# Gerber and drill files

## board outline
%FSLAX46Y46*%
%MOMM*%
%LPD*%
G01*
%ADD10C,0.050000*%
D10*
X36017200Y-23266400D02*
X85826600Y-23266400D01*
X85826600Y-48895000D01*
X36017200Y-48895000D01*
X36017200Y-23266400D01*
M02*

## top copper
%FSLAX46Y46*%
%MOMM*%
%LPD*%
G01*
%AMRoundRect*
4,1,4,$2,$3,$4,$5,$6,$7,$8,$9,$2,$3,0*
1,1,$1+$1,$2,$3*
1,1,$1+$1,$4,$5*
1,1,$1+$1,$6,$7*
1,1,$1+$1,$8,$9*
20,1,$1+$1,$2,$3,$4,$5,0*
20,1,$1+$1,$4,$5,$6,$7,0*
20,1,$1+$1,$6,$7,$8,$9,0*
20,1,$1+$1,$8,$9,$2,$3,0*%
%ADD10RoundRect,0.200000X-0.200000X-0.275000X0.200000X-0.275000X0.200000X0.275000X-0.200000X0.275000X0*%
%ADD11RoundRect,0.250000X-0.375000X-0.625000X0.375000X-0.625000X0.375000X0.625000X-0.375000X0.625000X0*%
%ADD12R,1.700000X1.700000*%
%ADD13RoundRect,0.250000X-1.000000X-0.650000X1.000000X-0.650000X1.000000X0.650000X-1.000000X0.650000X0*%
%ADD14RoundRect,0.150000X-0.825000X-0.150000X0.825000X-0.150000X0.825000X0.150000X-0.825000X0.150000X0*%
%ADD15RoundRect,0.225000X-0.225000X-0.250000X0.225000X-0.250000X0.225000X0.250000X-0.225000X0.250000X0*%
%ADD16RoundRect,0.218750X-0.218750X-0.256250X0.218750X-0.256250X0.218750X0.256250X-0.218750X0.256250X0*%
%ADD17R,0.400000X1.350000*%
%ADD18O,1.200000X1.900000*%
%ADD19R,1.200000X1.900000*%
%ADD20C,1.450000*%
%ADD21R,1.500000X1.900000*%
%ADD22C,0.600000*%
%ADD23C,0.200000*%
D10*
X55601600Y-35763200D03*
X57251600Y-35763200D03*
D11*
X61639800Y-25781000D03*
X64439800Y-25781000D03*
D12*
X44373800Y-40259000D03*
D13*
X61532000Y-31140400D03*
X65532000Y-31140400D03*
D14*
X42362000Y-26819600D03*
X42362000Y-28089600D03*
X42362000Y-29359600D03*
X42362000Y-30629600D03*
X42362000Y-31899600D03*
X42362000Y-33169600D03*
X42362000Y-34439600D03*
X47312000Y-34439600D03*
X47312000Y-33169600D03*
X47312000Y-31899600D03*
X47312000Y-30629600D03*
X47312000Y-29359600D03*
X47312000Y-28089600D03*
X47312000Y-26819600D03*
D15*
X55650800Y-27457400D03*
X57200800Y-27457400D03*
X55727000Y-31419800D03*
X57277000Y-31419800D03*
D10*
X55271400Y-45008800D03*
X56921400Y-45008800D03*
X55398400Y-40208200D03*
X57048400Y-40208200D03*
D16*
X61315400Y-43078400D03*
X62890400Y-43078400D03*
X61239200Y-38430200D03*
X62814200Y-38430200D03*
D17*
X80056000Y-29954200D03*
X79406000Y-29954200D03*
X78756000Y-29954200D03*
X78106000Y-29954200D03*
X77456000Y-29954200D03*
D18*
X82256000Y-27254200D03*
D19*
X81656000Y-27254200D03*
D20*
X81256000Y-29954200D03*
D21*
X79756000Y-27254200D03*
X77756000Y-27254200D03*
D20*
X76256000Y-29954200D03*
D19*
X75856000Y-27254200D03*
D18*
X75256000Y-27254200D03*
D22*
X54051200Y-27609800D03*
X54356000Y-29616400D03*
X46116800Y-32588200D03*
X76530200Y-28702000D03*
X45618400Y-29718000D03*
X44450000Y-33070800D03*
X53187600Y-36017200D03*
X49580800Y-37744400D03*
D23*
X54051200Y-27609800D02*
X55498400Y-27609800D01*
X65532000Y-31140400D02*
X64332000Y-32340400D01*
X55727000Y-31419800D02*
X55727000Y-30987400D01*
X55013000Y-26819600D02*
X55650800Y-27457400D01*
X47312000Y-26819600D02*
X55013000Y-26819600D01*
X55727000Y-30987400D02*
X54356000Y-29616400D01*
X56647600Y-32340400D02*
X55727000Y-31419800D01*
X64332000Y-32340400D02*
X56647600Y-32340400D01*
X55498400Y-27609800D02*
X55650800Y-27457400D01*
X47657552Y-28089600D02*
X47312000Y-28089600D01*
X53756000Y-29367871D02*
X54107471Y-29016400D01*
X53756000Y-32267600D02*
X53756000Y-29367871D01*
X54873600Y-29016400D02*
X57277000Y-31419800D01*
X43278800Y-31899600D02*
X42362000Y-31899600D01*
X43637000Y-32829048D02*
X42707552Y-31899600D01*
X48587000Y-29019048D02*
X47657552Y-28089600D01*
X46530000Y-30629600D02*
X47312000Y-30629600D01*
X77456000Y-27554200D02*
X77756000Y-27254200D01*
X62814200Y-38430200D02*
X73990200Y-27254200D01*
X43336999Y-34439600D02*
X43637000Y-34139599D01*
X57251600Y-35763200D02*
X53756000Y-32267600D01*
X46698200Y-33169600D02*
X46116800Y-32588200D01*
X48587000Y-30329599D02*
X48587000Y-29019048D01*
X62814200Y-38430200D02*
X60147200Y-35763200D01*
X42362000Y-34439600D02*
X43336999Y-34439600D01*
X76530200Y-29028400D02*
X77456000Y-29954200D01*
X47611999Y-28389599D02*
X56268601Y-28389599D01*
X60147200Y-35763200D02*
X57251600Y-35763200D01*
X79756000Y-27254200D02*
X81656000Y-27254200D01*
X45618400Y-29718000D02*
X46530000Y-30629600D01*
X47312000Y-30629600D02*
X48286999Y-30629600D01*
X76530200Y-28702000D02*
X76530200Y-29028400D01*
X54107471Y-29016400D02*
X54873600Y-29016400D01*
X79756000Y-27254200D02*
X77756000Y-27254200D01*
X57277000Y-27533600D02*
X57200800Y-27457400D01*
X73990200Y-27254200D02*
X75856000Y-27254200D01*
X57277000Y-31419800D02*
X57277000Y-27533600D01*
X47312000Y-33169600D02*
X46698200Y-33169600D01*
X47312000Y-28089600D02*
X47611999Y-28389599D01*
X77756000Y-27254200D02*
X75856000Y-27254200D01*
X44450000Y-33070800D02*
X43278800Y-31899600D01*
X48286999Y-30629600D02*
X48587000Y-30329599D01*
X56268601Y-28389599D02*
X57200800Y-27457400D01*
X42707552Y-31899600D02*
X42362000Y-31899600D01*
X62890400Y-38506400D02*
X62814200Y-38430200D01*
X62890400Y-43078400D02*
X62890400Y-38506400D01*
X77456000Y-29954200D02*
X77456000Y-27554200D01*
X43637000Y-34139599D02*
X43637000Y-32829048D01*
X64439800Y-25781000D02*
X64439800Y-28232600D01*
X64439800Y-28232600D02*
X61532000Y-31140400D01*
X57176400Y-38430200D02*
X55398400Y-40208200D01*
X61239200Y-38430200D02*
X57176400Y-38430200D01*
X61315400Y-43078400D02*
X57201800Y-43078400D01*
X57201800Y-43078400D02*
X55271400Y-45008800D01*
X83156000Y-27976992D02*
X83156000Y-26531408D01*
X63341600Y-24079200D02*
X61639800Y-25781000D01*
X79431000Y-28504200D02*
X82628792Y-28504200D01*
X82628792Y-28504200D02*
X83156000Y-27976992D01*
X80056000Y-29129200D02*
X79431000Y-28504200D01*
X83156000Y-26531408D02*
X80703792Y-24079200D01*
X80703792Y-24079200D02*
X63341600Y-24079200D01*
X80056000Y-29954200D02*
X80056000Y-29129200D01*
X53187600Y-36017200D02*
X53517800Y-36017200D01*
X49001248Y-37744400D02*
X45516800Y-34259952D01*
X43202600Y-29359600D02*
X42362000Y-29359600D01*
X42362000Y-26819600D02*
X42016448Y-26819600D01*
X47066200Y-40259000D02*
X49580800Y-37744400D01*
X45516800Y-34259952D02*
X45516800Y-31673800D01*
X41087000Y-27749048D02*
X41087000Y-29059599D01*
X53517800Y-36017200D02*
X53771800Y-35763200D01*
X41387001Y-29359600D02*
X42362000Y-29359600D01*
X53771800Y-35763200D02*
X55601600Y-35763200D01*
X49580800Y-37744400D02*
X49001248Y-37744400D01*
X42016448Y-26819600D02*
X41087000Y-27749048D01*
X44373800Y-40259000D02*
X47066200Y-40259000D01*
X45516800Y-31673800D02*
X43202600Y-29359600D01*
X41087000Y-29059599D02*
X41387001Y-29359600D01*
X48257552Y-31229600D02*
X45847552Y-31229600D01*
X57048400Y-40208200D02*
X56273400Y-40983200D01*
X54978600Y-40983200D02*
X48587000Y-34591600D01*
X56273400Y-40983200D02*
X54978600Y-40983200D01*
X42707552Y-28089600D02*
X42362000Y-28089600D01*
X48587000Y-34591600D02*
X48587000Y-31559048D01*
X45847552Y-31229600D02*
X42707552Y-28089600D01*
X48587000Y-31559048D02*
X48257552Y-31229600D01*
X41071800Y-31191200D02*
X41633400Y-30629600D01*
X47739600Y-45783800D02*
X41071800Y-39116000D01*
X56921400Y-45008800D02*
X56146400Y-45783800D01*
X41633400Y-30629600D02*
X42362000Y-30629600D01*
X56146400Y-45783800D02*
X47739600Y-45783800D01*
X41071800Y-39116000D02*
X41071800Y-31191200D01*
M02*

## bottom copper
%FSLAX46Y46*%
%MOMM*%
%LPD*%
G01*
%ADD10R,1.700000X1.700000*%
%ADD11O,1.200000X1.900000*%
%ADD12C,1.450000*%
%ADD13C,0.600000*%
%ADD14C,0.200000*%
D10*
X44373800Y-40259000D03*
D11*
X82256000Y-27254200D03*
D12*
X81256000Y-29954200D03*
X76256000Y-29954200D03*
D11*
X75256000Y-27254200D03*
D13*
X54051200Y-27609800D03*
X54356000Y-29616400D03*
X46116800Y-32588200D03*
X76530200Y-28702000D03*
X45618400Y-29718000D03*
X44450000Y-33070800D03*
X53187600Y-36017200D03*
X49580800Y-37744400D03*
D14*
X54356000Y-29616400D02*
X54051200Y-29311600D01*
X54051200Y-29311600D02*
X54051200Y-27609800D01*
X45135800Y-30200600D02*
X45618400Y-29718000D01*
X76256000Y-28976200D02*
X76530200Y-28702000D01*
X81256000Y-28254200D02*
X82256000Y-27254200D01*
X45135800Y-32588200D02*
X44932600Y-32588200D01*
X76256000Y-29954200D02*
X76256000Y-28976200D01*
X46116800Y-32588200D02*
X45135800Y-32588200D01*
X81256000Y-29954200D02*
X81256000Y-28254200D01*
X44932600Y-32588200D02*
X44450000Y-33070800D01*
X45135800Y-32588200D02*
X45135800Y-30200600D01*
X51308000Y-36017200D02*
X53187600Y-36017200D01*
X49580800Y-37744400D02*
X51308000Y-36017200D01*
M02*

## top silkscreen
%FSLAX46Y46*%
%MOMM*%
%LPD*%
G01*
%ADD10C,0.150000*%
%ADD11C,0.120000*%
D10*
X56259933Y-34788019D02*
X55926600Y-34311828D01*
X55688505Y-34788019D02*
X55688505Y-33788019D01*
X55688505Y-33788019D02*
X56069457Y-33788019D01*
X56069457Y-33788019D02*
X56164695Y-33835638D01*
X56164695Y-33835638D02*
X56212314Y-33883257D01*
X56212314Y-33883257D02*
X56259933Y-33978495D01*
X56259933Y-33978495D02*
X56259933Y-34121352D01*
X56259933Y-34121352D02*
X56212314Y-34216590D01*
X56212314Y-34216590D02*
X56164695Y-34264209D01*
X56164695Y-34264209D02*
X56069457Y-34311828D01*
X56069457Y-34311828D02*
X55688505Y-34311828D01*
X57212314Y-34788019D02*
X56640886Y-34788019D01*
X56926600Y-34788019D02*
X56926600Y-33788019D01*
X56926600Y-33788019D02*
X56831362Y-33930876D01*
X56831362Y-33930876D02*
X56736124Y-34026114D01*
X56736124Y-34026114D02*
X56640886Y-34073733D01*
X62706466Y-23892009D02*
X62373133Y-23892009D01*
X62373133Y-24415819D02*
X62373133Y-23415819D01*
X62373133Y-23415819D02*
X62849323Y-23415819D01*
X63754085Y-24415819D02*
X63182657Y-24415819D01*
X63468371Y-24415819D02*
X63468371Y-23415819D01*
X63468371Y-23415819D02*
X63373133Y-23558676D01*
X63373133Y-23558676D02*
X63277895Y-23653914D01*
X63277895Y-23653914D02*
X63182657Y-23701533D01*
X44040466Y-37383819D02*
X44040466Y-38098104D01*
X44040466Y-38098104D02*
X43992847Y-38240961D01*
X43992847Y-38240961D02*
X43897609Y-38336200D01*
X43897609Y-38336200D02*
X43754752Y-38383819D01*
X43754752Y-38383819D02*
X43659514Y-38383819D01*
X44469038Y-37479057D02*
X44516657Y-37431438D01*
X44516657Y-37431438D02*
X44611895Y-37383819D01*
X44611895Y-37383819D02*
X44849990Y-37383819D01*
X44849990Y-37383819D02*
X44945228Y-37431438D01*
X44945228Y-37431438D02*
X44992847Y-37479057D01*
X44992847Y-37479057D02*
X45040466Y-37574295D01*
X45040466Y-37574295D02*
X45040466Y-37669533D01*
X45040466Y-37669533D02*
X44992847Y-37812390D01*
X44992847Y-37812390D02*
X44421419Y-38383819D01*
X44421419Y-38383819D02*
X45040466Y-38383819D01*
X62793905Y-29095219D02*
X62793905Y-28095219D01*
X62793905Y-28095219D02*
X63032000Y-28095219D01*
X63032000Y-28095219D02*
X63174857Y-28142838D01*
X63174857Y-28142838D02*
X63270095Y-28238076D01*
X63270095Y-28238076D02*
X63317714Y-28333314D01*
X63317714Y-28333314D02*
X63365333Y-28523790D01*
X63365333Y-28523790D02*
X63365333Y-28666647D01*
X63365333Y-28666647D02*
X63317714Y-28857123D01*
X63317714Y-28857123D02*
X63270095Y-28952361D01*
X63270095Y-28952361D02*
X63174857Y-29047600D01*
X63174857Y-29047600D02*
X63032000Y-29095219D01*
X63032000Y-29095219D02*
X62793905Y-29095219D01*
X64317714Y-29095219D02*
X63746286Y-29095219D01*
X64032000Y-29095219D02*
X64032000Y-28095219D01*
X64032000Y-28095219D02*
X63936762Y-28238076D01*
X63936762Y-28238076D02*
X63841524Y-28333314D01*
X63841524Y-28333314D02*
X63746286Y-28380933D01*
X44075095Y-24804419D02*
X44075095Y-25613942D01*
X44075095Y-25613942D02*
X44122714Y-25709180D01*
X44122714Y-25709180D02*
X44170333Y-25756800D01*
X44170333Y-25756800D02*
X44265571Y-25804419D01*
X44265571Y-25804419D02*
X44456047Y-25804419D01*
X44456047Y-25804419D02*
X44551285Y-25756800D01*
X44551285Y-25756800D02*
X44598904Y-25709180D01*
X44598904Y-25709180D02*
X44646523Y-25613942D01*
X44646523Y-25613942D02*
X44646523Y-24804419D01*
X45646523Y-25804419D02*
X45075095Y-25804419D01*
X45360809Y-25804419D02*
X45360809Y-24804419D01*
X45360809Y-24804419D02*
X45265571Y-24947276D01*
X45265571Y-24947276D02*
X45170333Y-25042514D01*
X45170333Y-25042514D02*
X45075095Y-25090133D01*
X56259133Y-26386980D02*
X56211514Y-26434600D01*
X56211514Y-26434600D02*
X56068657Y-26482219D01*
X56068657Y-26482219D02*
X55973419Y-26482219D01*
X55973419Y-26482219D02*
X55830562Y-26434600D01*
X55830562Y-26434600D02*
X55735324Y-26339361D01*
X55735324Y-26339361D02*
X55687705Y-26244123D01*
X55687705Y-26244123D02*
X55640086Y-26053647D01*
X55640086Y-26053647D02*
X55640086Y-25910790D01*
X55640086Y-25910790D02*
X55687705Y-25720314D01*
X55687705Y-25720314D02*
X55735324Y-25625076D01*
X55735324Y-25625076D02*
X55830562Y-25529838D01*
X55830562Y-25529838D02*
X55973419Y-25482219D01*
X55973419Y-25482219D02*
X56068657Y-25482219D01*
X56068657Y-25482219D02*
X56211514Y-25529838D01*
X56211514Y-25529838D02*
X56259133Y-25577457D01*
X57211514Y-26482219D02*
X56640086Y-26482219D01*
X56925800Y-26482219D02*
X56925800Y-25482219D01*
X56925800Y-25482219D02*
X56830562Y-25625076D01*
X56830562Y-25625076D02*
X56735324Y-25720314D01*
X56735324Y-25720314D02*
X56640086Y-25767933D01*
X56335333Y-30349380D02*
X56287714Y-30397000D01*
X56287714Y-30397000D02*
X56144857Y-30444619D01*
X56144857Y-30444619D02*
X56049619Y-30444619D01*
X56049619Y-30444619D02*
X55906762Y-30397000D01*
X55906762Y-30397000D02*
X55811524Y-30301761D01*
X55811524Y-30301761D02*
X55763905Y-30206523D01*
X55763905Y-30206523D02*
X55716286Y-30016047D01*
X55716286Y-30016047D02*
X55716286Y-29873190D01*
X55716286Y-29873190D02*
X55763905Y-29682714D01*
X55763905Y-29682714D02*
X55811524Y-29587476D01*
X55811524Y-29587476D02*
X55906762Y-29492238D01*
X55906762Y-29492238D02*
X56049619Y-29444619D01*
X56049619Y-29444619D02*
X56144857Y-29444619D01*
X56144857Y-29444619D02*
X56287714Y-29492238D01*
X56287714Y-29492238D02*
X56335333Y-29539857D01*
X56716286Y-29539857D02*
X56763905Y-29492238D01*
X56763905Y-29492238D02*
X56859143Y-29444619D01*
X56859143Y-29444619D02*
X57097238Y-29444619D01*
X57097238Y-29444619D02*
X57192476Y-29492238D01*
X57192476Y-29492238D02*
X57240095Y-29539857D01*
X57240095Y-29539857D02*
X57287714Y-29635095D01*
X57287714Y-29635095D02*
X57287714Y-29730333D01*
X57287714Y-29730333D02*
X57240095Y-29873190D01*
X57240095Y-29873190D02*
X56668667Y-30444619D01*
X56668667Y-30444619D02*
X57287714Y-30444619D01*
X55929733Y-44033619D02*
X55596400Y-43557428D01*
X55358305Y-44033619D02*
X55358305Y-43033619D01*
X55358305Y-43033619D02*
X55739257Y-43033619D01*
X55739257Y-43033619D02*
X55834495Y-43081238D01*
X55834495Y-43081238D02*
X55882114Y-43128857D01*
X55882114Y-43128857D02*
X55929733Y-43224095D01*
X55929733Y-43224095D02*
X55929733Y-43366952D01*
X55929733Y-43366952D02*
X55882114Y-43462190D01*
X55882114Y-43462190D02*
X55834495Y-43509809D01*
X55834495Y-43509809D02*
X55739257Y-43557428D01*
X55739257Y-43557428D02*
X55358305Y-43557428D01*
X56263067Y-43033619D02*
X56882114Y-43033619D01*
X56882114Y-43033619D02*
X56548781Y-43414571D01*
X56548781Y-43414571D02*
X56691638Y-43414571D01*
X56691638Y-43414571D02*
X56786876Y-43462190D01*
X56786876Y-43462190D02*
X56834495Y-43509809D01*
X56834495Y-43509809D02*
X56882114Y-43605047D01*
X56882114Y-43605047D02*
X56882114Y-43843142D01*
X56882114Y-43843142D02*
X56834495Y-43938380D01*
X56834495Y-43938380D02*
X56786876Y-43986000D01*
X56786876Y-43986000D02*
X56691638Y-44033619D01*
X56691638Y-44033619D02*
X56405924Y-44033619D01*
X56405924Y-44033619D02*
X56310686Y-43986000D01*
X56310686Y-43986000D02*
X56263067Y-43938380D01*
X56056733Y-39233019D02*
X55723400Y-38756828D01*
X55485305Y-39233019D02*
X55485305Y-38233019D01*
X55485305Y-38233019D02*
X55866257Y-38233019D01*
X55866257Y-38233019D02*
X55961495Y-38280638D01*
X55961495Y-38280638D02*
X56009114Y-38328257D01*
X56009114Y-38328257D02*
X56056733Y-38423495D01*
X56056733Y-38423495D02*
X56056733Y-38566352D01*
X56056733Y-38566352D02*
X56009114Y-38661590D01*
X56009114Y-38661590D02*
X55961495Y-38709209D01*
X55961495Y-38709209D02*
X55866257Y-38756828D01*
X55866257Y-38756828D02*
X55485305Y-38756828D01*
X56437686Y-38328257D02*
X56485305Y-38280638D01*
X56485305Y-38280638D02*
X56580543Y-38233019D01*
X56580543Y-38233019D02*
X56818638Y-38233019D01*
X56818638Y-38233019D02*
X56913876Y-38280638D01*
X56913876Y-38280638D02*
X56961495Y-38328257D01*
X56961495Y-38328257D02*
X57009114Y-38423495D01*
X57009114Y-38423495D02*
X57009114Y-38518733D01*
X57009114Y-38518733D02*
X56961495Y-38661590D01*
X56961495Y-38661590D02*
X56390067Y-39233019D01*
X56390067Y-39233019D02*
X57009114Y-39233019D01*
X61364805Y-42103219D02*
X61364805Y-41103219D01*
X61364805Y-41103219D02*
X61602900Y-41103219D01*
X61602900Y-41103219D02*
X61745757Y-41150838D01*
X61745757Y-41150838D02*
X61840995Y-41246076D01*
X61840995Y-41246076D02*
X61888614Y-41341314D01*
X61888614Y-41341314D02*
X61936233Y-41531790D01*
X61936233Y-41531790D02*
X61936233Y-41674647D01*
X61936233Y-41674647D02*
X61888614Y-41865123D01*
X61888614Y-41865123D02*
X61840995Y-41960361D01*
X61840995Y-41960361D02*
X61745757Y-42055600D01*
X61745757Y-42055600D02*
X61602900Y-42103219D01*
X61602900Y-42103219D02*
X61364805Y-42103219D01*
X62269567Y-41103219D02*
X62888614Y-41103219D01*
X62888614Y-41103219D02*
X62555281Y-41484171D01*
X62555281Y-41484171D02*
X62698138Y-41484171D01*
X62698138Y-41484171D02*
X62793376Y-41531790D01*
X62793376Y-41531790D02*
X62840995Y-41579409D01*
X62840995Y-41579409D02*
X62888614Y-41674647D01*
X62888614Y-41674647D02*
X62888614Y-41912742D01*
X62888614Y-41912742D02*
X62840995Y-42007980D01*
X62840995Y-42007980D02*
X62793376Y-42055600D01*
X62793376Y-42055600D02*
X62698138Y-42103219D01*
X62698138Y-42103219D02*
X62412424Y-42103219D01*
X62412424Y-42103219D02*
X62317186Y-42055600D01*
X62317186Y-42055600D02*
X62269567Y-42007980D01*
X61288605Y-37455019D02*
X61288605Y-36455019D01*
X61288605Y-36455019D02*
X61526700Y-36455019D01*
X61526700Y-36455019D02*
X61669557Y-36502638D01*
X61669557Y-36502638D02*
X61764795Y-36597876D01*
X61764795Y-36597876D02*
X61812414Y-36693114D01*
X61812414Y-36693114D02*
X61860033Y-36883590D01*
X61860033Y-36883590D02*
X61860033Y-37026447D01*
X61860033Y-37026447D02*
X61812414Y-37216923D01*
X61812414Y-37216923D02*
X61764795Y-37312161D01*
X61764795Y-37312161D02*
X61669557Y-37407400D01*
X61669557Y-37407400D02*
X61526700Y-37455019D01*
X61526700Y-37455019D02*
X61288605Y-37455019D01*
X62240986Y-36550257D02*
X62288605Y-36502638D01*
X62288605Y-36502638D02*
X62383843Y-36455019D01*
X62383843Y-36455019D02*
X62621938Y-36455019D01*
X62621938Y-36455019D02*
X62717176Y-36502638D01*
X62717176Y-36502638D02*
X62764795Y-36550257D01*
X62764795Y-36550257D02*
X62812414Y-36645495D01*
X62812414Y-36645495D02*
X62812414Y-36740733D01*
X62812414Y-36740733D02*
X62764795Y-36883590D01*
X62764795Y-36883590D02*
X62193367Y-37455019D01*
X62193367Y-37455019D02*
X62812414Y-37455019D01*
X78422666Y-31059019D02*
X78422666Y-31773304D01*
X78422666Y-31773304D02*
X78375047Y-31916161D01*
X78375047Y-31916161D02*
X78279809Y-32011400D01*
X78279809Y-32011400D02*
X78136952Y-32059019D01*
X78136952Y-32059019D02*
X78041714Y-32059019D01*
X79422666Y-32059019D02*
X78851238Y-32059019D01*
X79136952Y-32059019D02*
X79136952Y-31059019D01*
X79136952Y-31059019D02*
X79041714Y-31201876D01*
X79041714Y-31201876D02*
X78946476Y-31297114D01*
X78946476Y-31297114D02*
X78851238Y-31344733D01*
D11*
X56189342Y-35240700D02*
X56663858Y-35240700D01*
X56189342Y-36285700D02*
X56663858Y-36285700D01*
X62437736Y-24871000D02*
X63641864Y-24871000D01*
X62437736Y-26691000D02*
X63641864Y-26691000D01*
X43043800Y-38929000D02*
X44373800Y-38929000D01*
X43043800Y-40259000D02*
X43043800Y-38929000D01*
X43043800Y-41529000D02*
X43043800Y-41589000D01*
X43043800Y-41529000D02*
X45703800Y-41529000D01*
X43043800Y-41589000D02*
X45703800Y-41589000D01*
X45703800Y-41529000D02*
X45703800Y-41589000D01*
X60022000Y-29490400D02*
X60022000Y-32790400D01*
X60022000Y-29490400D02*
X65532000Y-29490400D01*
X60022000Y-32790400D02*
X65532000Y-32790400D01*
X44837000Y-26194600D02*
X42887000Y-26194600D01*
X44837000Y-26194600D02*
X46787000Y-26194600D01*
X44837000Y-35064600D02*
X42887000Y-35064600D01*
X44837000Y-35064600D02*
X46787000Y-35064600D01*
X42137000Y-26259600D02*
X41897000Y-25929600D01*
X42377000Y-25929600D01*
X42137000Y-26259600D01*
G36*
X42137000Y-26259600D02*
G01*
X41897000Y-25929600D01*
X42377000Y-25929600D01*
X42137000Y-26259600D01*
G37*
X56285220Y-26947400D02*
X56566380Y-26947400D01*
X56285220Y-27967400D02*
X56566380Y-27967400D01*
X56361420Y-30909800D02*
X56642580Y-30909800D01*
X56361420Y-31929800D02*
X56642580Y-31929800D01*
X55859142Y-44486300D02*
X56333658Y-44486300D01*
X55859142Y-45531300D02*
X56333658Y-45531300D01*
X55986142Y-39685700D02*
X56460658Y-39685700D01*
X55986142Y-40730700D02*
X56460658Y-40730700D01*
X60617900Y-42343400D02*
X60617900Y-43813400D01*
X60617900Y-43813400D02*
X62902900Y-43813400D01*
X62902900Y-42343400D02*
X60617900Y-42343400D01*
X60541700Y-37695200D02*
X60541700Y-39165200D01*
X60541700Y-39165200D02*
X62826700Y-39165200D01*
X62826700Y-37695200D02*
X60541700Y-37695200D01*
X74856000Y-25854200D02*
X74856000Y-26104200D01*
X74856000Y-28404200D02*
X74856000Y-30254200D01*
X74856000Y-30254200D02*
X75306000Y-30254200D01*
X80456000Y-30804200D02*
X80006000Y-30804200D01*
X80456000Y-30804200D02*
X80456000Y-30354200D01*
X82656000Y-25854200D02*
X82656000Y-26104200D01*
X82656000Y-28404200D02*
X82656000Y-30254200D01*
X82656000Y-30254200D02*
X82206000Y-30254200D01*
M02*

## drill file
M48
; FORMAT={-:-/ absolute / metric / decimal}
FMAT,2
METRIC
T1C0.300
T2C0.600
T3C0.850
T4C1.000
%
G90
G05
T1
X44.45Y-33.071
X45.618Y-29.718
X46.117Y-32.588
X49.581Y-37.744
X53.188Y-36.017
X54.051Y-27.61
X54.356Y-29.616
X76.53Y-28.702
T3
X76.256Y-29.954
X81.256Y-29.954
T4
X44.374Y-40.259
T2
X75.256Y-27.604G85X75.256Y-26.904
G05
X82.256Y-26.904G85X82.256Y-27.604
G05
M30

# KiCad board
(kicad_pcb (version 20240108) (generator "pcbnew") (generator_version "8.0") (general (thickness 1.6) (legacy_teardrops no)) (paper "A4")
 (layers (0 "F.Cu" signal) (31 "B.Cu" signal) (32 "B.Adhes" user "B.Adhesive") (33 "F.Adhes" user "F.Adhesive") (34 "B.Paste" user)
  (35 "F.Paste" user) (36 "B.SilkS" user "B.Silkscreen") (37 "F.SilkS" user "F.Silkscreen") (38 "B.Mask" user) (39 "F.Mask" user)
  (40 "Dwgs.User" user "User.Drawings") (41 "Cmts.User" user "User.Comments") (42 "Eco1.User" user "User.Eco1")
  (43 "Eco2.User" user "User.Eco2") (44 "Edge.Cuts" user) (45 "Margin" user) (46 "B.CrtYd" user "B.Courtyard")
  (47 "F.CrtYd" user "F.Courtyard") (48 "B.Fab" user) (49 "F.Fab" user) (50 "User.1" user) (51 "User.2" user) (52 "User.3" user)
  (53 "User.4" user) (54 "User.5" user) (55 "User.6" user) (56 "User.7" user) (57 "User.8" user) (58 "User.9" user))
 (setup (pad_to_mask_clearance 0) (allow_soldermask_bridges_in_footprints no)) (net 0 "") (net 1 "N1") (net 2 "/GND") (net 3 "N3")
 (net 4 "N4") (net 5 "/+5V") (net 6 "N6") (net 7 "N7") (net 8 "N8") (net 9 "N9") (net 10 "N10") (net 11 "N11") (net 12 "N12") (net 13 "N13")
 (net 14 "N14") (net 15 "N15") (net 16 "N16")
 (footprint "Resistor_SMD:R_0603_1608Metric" (layer "F.Cu") (at 56.4266 35.7632)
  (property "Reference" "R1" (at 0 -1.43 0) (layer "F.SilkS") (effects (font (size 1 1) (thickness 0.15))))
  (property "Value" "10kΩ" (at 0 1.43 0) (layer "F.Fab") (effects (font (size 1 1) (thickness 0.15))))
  (fp_line (start -0.237258 -0.5225) (end 0.237258 -0.5225) (stroke (width 0.12) (type solid)) (layer "F.SilkS"))
  (fp_line (start -0.237258 0.5225) (end 0.237258 0.5225) (stroke (width 0.12) (type solid)) (layer "F.SilkS"))
  (pad "1" smd roundrect (at -0.825 0) (size 0.8 0.95) (layers "F.Cu" "F.Paste" "F.Mask") (roundrect_rratio 0.25) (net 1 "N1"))
  (pad "2" smd roundrect (at 0.825 0) (size 0.8 0.95) (layers "F.Cu" "F.Paste" "F.Mask") (roundrect_rratio 0.25) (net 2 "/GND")))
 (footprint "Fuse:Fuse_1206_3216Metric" (layer "F.Cu") (at 63.0398 25.781)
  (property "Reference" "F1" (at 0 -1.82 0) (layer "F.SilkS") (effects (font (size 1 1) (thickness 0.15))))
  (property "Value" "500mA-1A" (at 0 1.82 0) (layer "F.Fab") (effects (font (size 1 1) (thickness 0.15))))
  (fp_line (start -0.602064 -0.91) (end 0.602064 -0.91) (stroke (width 0.12) (type solid)) (layer "F.SilkS"))
  (fp_line (start -0.602064 0.91) (end 0.602064 0.91) (stroke (width 0.12) (type solid)) (layer "F.SilkS"))
  (pad "1" smd roundrect (at -1.4 0) (size 1.25 1.75) (layers "F.Cu" "F.Paste" "F.Mask") (roundrect_rratio 0.2) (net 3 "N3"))
  (pad "2" smd roundrect (at 1.4 0) (size 1.25 1.75) (layers "F.Cu" "F.Paste" "F.Mask") (roundrect_rratio 0.2) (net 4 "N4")))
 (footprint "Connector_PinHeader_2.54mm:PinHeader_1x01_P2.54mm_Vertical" (layer "F.Cu") (at 44.3738 40.259)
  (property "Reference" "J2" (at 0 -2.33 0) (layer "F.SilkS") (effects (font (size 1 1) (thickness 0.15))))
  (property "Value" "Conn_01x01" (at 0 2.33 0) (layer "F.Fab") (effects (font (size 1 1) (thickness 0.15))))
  (fp_line (start -1.33 -1.33) (end 0 -1.33) (stroke (width 0.12) (type solid)) (layer "F.SilkS"))
  (fp_line (start -1.33 0) (end -1.33 -1.33) (stroke (width 0.12) (type solid)) (layer "F.SilkS"))
  (fp_line (start -1.33 1.27) (end -1.33 1.33) (stroke (width 0.12) (type solid)) (layer "F.SilkS"))
  (fp_line (start -1.33 1.27) (end 1.33 1.27) (stroke (width 0.12) (type solid)) (layer "F.SilkS"))
  (fp_line (start -1.33 1.33) (end 1.33 1.33) (stroke (width 0.12) (type solid)) (layer "F.SilkS"))
  (fp_line (start 1.33 1.27) (end 1.33 1.33) (stroke (width 0.12) (type solid)) (layer "F.SilkS"))
  (pad "1" thru_hole rect (at 0 0) (size 1.7 1.7) (drill 1) (layers "*.Cu" "*.Mask") (remove_unused_layers no) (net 1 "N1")))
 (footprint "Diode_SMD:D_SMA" (layer "F.Cu") (at 63.532 31.1404)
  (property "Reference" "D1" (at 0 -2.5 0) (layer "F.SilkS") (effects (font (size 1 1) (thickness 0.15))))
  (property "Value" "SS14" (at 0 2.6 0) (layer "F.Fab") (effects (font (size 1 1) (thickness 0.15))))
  (fp_line (start -3.51 -1.65) (end -3.51 1.65) (stroke (width 0.12) (type solid)) (layer "F.SilkS"))
  (fp_line (start -3.51 -1.65) (end 2 -1.65) (stroke (width 0.12) (type solid)) (layer "F.SilkS"))
  (fp_line (start -3.51 1.65) (end 2 1.65) (stroke (width 0.12) (type solid)) (layer "F.SilkS"))
  (pad "1" smd roundrect (at -2 0) (size 2.5 1.8) (layers "F.Cu" "F.Paste" "F.Mask") (roundrect_rratio 0.1388888889) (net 4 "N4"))
  (pad "2" smd roundrect (at 2 0) (size 2.5 1.8) (layers "F.Cu" "F.Paste" "F.Mask") (roundrect_rratio 0.1388888889) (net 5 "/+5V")))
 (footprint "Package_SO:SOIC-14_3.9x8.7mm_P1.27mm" (layer "F.Cu") (at 44.837 30.6296)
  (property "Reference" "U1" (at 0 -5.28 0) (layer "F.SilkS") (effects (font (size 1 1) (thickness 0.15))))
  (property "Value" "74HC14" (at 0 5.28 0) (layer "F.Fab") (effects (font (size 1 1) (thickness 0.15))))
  (fp_line (start 0 -4.435) (end -1.95 -4.435) (stroke (width 0.12) (type solid)) (layer "F.SilkS"))
  (fp_line (start 0 -4.435) (end 1.95 -4.435) (stroke (width 0.12) (type solid)) (layer "F.SilkS"))
  (fp_line (start 0 4.435) (end -1.95 4.435) (stroke (width 0.12) (type solid)) (layer "F.SilkS"))
  (fp_line (start 0 4.435) (end 1.95 4.435) (stroke (width 0.12) (type solid)) (layer "F.SilkS"))
  (fp_poly
   (pts (xy -2.7 -4.37) (xy -2.94 -4.7) (xy -2.46 -4.7) (xy -2.7 -4.37)) (stroke (width 0.12) (type solid)) (fill solid) (layer "F.SilkS"))
  (pad "1" smd roundrect (at -2.475 -3.81) (size 1.95 0.6) (layers "F.Cu" "F.Paste" "F.Mask") (roundrect_rratio 0.25) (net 1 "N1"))
  (pad "2" smd roundrect (at -2.475 -2.54) (size 1.95 0.6) (layers "F.Cu" "F.Paste" "F.Mask") (roundrect_rratio 0.25) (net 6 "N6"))
  (pad "3" smd roundrect (at -2.475 -1.27) (size 1.95 0.6) (layers "F.Cu" "F.Paste" "F.Mask") (roundrect_rratio 0.25) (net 1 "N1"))
  (pad "4" smd roundrect (at -2.475 0) (size 1.95 0.6) (layers "F.Cu" "F.Paste" "F.Mask") (roundrect_rratio 0.25) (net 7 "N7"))
  (pad "5" smd roundrect (at -2.475 1.27) (size 1.95 0.6) (layers "F.Cu" "F.Paste" "F.Mask") (roundrect_rratio 0.25) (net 2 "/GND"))
  (pad "6" smd roundrect (at -2.475 2.54) (size 1.95 0.6) (layers "F.Cu" "F.Paste" "F.Mask") (roundrect_rratio 0.25) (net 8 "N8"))
  (pad "7" smd roundrect (at -2.475 3.81) (size 1.95 0.6) (layers "F.Cu" "F.Paste" "F.Mask") (roundrect_rratio 0.25) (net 2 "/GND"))
  (pad "8" smd roundrect (at 2.475 3.81) (size 1.95 0.6) (layers "F.Cu" "F.Paste" "F.Mask") (roundrect_rratio 0.25) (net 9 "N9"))
  (pad "9" smd roundrect (at 2.475 2.54) (size 1.95 0.6) (layers "F.Cu" "F.Paste" "F.Mask") (roundrect_rratio 0.25) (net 2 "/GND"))
  (pad "10" smd roundrect (at 2.475 1.27) (size 1.95 0.6) (layers "F.Cu" "F.Paste" "F.Mask") (roundrect_rratio 0.25) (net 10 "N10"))
  (pad "11" smd roundrect (at 2.475 0) (size 1.95 0.6) (layers "F.Cu" "F.Paste" "F.Mask") (roundrect_rratio 0.25) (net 2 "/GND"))
  (pad "12" smd roundrect (at 2.475 -1.27) (size 1.95 0.6) (layers "F.Cu" "F.Paste" "F.Mask") (roundrect_rratio 0.25) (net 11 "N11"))
  (pad "13" smd roundrect (at 2.475 -2.54) (size 1.95 0.6) (layers "F.Cu" "F.Paste" "F.Mask") (roundrect_rratio 0.25) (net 2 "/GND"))
  (pad "14" smd roundrect (at 2.475 -3.81) (size 1.95 0.6) (layers "F.Cu" "F.Paste" "F.Mask") (roundrect_rratio 0.25) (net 5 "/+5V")))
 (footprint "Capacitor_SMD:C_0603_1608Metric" (layer "F.Cu") (at 56.4258 27.4574)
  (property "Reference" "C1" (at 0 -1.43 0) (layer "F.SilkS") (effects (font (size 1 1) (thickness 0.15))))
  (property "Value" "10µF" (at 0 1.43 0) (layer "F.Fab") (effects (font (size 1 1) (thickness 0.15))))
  (fp_line (start -0.14058 -0.51) (end 0.14058 -0.51) (stroke (width 0.12) (type solid)) (layer "F.SilkS"))
  (fp_line (start -0.14058 0.51) (end 0.14058 0.51) (stroke (width 0.12) (type solid)) (layer "F.SilkS"))
  (pad "1" smd roundrect (at -0.775 0) (size 0.9 0.95) (layers "F.Cu" "F.Paste" "F.Mask") (roundrect_rratio 0.25) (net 5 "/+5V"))
  (pad "2" smd roundrect (at 0.775 0) (size 0.9 0.95) (layers "F.Cu" "F.Paste" "F.Mask") (roundrect_rratio 0.25) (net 2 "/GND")))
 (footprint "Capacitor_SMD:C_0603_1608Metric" (layer "F.Cu") (at 56.502 31.4198)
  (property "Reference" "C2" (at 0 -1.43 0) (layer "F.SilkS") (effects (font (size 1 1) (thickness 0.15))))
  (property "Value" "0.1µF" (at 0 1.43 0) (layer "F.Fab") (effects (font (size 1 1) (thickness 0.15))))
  (fp_line (start -0.14058 -0.51) (end 0.14058 -0.51) (stroke (width 0.12) (type solid)) (layer "F.SilkS"))
  (fp_line (start -0.14058 0.51) (end 0.14058 0.51) (stroke (width 0.12) (type solid)) (layer "F.SilkS"))
  (pad "1" smd roundrect (at -0.775 0) (size 0.9 0.95) (layers "F.Cu" "F.Paste" "F.Mask") (roundrect_rratio 0.25) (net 5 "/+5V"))
  (pad "2" smd roundrect (at 0.775 0) (size 0.9 0.95) (layers "F.Cu" "F.Paste" "F.Mask") (roundrect_rratio 0.25) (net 2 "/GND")))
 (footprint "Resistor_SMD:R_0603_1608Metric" (layer "F.Cu") (at 56.0964 45.0088)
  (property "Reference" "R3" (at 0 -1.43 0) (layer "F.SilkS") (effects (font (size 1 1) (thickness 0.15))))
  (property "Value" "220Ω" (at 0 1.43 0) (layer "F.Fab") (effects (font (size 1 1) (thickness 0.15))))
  (fp_line (start -0.237258 -0.5225) (end 0.237258 -0.5225) (stroke (width 0.12) (type solid)) (layer "F.SilkS"))
  (fp_line (start -0.237258 0.5225) (end 0.237258 0.5225) (stroke (width 0.12) (type solid)) (layer "F.SilkS"))
  (pad "1" smd roundrect (at -0.825 0) (size 0.8 0.95) (layers "F.Cu" "F.Paste" "F.Mask") (roundrect_rratio 0.25) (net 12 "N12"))
  (pad "2" smd roundrect (at 0.825 0) (size 0.8 0.95) (layers "F.Cu" "F.Paste" "F.Mask") (roundrect_rratio 0.25) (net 7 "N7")))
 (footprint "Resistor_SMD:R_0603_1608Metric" (layer "F.Cu") (at 56.2234 40.2082)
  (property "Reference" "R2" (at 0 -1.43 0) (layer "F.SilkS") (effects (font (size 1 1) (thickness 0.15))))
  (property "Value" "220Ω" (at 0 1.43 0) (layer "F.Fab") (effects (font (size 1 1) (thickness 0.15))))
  (fp_line (start -0.237258 -0.5225) (end 0.237258 -0.5225) (stroke (width 0.12) (type solid)) (layer "F.SilkS"))
  (fp_line (start -0.237258 0.5225) (end 0.237258 0.5225) (stroke (width 0.12) (type solid)) (layer "F.SilkS"))
  (pad "1" smd roundrect (at -0.825 0) (size 0.8 0.95) (layers "F.Cu" "F.Paste" "F.Mask") (roundrect_rratio 0.25) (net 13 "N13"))
  (pad "2" smd roundrect (at 0.825 0) (size 0.8 0.95) (layers "F.Cu" "F.Paste" "F.Mask") (roundrect_rratio 0.25) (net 6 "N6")))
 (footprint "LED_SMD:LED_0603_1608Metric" (layer "F.Cu") (at 62.1029 43.0784)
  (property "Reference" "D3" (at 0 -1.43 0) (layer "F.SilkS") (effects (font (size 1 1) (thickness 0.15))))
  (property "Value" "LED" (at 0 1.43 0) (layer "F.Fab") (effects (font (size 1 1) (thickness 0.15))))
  (fp_line (start -1.485 -0.735) (end -1.485 0.735) (stroke (width 0.12) (type solid)) (layer "F.SilkS"))
  (fp_line (start -1.485 0.735) (end 0.8 0.735) (stroke (width 0.12) (type solid)) (layer "F.SilkS"))
  (fp_line (start 0.8 -0.735) (end -1.485 -0.735) (stroke (width 0.12) (type solid)) (layer "F.SilkS"))
  (pad "1" smd roundrect (at -0.7875 0) (size 0.875 0.95) (layers "F.Cu" "F.Paste" "F.Mask") (roundrect_rratio 0.25) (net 12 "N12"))
  (pad "2" smd roundrect (at 0.7875 0) (size 0.875 0.95) (layers "F.Cu" "F.Paste" "F.Mask") (roundrect_rratio 0.25) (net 2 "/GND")))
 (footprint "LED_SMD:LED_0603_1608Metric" (layer "F.Cu") (at 62.0267 38.4302)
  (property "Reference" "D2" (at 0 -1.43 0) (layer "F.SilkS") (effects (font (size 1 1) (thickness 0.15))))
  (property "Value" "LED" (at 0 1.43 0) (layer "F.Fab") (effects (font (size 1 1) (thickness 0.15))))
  (fp_line (start -1.485 -0.735) (end -1.485 0.735) (stroke (width 0.12) (type solid)) (layer "F.SilkS"))
  (fp_line (start -1.485 0.735) (end 0.8 0.735) (stroke (width 0.12) (type solid)) (layer "F.SilkS"))
  (fp_line (start 0.8 -0.735) (end -1.485 -0.735) (stroke (width 0.12) (type solid)) (layer "F.SilkS"))
  (pad "1" smd roundrect (at -0.7875 0) (size 0.875 0.95) (layers "F.Cu" "F.Paste" "F.Mask") (roundrect_rratio 0.25) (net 13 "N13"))
  (pad "2" smd roundrect (at 0.7875 0) (size 0.875 0.95) (layers "F.Cu" "F.Paste" "F.Mask") (roundrect_rratio 0.25) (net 2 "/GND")))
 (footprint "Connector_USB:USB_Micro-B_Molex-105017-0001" (layer "F.Cu") (at 78.756 28.4917 180)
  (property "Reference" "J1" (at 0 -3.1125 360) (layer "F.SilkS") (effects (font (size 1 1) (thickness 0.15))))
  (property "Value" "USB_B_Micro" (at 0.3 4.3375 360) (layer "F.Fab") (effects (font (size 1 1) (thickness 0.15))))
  (fp_line (start 3.9 2.6375) (end 3.9 2.3875) (stroke (width 0.12) (type solid)) (layer "F.SilkS"))
  (fp_line (start 3.9 0.0875) (end 3.9 -1.7625) (stroke (width 0.12) (type solid)) (layer "F.SilkS"))
  (fp_line (start 3.9 -1.7625) (end 3.45 -1.7625) (stroke (width 0.12) (type solid)) (layer "F.SilkS"))
  (fp_line (start -1.7 -2.3125) (end -1.25 -2.3125) (stroke (width 0.12) (type solid)) (layer "F.SilkS"))
  (fp_line (start -1.7 -2.3125) (end -1.7 -1.8625) (stroke (width 0.12) (type solid)) (layer "F.SilkS"))
  (fp_line (start -3.9 2.6375) (end -3.9 2.3875) (stroke (width 0.12) (type solid)) (layer "F.SilkS"))
  (fp_line (start -3.9 0.0875) (end -3.9 -1.7625) (stroke (width 0.12) (type solid)) (layer "F.SilkS"))
  (fp_line (start -3.9 -1.7625) (end -3.45 -1.7625) (stroke (width 0.12) (type solid)) (layer "F.SilkS"))
  (pad "1" smd rect (at -1.3 -1.4625 180) (size 0.4 1.35) (layers "F.Cu" "F.Paste" "F.Mask") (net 3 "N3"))
  (pad "2" smd rect (at -0.65 -1.4625 180) (size 0.4 1.35) (layers "F.Cu" "F.Paste" "F.Mask") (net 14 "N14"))
  (pad "3" smd rect (at 0 -1.4625 180) (size 0.4 1.35) (layers "F.Cu" "F.Paste" "F.Mask") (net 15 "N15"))
  (pad "4" smd rect (at 0.65 -1.4625 180) (size 0.4 1.35) (layers "F.Cu" "F.Paste" "F.Mask") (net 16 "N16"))
  (pad "5" smd rect (at 1.3 -1.4625 180) (size 0.4 1.35) (layers "F.Cu" "F.Paste" "F.Mask") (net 2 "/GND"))
  (pad "6" thru_hole oval (at -3.5 1.2375) (size 1.2 1.9) (drill oval 0.6 1.3) (layers "*.Cu" "*.Mask") (remove_unused_layers no)
   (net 2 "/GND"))
  (pad "6" smd rect (at -2.9 1.2375 180) (size 1.2 1.9) (layers "F.Cu" "F.Mask") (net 2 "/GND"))
  (pad "6" thru_hole circle (at -2.5 -1.4625 180) (size 1.45 1.45) (drill 0.85) (layers "*.Cu" "*.Mask") (remove_unused_layers no)
   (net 2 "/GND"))
  (pad "6" smd rect (at -1 1.2375 180) (size 1.5 1.9) (layers "F.Cu" "F.Paste" "F.Mask") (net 2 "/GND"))
  (pad "6" smd rect (at 1 1.2375 180) (size 1.5 1.9) (layers "F.Cu" "F.Paste" "F.Mask") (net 2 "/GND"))
  (pad "6" thru_hole circle (at 2.5 -1.4625 180) (size 1.45 1.45) (drill 0.85) (layers "*.Cu" "*.Mask") (remove_unused_layers no)
   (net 2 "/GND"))
  (pad "6" smd rect (at 2.9 1.2375 180) (size 1.2 1.9) (layers "F.Cu" "F.Mask") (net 2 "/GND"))
  (pad "6" thru_hole oval (at 3.5 1.2375 180) (size 1.2 1.9) (drill oval 0.6 1.3) (layers "*.Cu" "*.Mask") (remove_unused_layers no)
   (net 2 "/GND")))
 (gr_rect (start 36.0172 23.2664) (end 85.8266 48.895) (stroke (width 0.05) (type default)) (fill none) (layer "Edge.Cuts"))
 (segment (start 54.0512 27.6098) (end 55.4984 27.6098) (width 0.2) (layer "F.Cu") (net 5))
 (segment (start 65.532 31.1404) (end 64.332 32.3404) (width 0.2) (layer "F.Cu") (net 5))
 (segment (start 55.727 31.4198) (end 55.727 30.9874) (width 0.2) (layer "F.Cu") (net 5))
 (segment (start 55.013 26.8196) (end 55.6508 27.4574) (width 0.2) (layer "F.Cu") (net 5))
 (segment (start 47.312 26.8196) (end 55.013 26.8196) (width 0.2) (layer "F.Cu") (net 5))
 (segment (start 55.727 30.9874) (end 54.356 29.6164) (width 0.2) (layer "F.Cu") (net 5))
 (segment (start 56.6476 32.3404) (end 55.727 31.4198) (width 0.2) (layer "F.Cu") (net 5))
 (segment (start 64.332 32.3404) (end 56.6476 32.3404) (width 0.2) (layer "F.Cu") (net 5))
 (segment (start 55.4984 27.6098) (end 55.6508 27.4574) (width 0.2) (layer "F.Cu") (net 5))
 (via (at 54.0512 27.6098) (size 0.6) (drill 0.3) (layers "F.Cu" "B.Cu") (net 5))
 (via (at 54.356 29.6164) (size 0.6) (drill 0.3) (layers "F.Cu" "B.Cu") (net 5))
 (segment (start 54.356 29.6164) (end 54.0512 29.3116) (width 0.2) (layer "B.Cu") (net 5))
 (segment (start 54.0512 29.3116) (end 54.0512 27.6098) (width 0.2) (layer "B.Cu") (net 5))
 (segment (start 47.657552 28.0896) (end 47.312 28.0896) (width 0.2) (layer "F.Cu") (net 2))
 (segment (start 53.756 29.367871) (end 54.107471 29.0164) (width 0.2) (layer "F.Cu") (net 2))
 (segment (start 53.756 32.2676) (end 53.756 29.367871) (width 0.2) (layer "F.Cu") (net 2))
 (segment (start 54.8736 29.0164) (end 57.277 31.4198) (width 0.2) (layer "F.Cu") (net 2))
 (segment (start 43.2788 31.8996) (end 42.362 31.8996) (width 0.2) (layer "F.Cu") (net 2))
 (segment (start 43.637 32.829048) (end 42.707552 31.8996) (width 0.2) (layer "F.Cu") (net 2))
 (segment (start 48.587 29.019048) (end 47.657552 28.0896) (width 0.2) (layer "F.Cu") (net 2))
 (segment (start 46.53 30.6296) (end 47.312 30.6296) (width 0.2) (layer "F.Cu") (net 2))
 (segment (start 77.456 27.5542) (end 77.756 27.2542) (width 0.2) (layer "F.Cu") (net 2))
 (segment (start 62.8142 38.4302) (end 73.9902 27.2542) (width 0.2) (layer "F.Cu") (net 2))
 (segment (start 43.336999 34.4396) (end 43.637 34.139599) (width 0.2) (layer "F.Cu") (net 2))
 (segment (start 57.2516 35.7632) (end 53.756 32.2676) (width 0.2) (layer "F.Cu") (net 2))
 (segment (start 46.6982 33.1696) (end 46.1168 32.5882) (width 0.2) (layer "F.Cu") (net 2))
 (segment (start 48.587 30.329599) (end 48.587 29.019048) (width 0.2) (layer "F.Cu") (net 2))
 (segment (start 62.8142 38.4302) (end 60.1472 35.7632) (width 0.2) (layer "F.Cu") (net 2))
 (segment (start 42.362 34.4396) (end 43.336999 34.4396) (width 0.2) (layer "F.Cu") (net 2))
 (segment (start 76.5302 29.0284) (end 77.456 29.9542) (width 0.2) (layer "F.Cu") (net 2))
 (segment (start 47.611999 28.389599) (end 56.268601 28.389599) (width 0.2) (layer "F.Cu") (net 2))
 (segment (start 60.1472 35.7632) (end 57.2516 35.7632) (width 0.2) (layer "F.Cu") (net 2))
 (segment (start 79.756 27.2542) (end 81.656 27.2542) (width 0.2) (layer "F.Cu") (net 2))
 (segment (start 45.6184 29.718) (end 46.53 30.6296) (width 0.2) (layer "F.Cu") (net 2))
 (segment (start 47.312 30.6296) (end 48.286999 30.6296) (width 0.2) (layer "F.Cu") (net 2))
 (segment (start 76.5302 28.702) (end 76.5302 29.0284) (width 0.2) (layer "F.Cu") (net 2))
 (segment (start 54.107471 29.0164) (end 54.8736 29.0164) (width 0.2) (layer "F.Cu") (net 2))
 (segment (start 79.756 27.2542) (end 77.756 27.2542) (width 0.2) (layer "F.Cu") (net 2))
 (segment (start 57.277 27.5336) (end 57.2008 27.4574) (width 0.2) (layer "F.Cu") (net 2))
 (segment (start 73.9902 27.2542) (end 75.856 27.2542) (width 0.2) (layer "F.Cu") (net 2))
 (segment (start 57.277 31.4198) (end 57.277 27.5336) (width 0.2) (layer "F.Cu") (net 2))
 (segment (start 47.312 33.1696) (end 46.6982 33.1696) (width 0.2) (layer "F.Cu") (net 2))
 (segment (start 47.312 28.0896) (end 47.611999 28.389599) (width 0.2) (layer "F.Cu") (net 2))
 (segment (start 77.756 27.2542) (end 75.856 27.2542) (width 0.2) (layer "F.Cu") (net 2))
 (segment (start 44.45 33.0708) (end 43.2788 31.8996) (width 0.2) (layer "F.Cu") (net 2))
 (segment (start 48.286999 30.6296) (end 48.587 30.329599) (width 0.2) (layer "F.Cu") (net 2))
 (segment (start 56.268601 28.389599) (end 57.2008 27.4574) (width 0.2) (layer "F.Cu") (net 2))
 (segment (start 42.707552 31.8996) (end 42.362 31.8996) (width 0.2) (layer "F.Cu") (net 2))
 (segment (start 62.8904 38.5064) (end 62.8142 38.4302) (width 0.2) (layer "F.Cu") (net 2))
 (segment (start 62.8904 43.0784) (end 62.8904 38.5064) (width 0.2) (layer "F.Cu") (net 2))
 (segment (start 77.456 29.9542) (end 77.456 27.5542) (width 0.2) (layer "F.Cu") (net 2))
 (segment (start 43.637 34.139599) (end 43.637 32.829048) (width 0.2) (layer "F.Cu") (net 2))
 (via (at 46.1168 32.5882) (size 0.6) (drill 0.3) (layers "F.Cu" "B.Cu") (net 2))
 (via (at 76.5302 28.702) (size 0.6) (drill 0.3) (layers "F.Cu" "B.Cu") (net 2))
 (via (at 45.6184 29.718) (size 0.6) (drill 0.3) (layers "F.Cu" "B.Cu") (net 2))
 (via (at 44.45 33.0708) (size 0.6) (drill 0.3) (layers "F.Cu" "B.Cu") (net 2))
 (segment (start 45.1358 30.2006) (end 45.6184 29.718) (width 0.2) (layer "B.Cu") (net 2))
 (segment (start 76.256 28.9762) (end 76.5302 28.702) (width 0.2) (layer "B.Cu") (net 2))
 (segment (start 81.256 28.2542) (end 82.256 27.2542) (width 0.2) (layer "B.Cu") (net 2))
 (segment (start 45.1358 32.5882) (end 44.9326 32.5882) (width 0.2) (layer "B.Cu") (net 2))
 (segment (start 76.256 29.9542) (end 76.256 28.9762) (width 0.2) (layer "B.Cu") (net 2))
 (segment (start 46.1168 32.5882) (end 45.1358 32.5882) (width 0.2) (layer "B.Cu") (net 2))
 (segment (start 81.256 29.9542) (end 81.256 28.2542) (width 0.2) (layer "B.Cu") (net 2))
 (segment (start 44.9326 32.5882) (end 44.45 33.0708) (width 0.2) (layer "B.Cu") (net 2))
 (segment (start 45.1358 32.5882) (end 45.1358 30.2006) (width 0.2) (layer "B.Cu") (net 2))
 (segment (start 64.4398 25.781) (end 64.4398 28.2326) (width 0.2) (layer "F.Cu") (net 4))
 (segment (start 64.4398 28.2326) (end 61.532 31.1404) (width 0.2) (layer "F.Cu") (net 4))
 (segment (start 57.1764 38.4302) (end 55.3984 40.2082) (width 0.2) (layer "F.Cu") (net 13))
 (segment (start 61.2392 38.4302) (end 57.1764 38.4302) (width 0.2) (layer "F.Cu") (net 13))
 (segment (start 61.3154 43.0784) (end 57.2018 43.0784) (width 0.2) (layer "F.Cu") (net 12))
 (segment (start 57.2018 43.0784) (end 55.2714 45.0088) (width 0.2) (layer "F.Cu") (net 12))
 (segment (start 83.156 27.976992) (end 83.156 26.531408) (width 0.2) (layer "F.Cu") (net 3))
 (segment (start 63.3416 24.0792) (end 61.6398 25.781) (width 0.2) (layer "F.Cu") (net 3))
 (segment (start 79.431 28.5042) (end 82.628792 28.5042) (width 0.2) (layer "F.Cu") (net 3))
 (segment (start 82.628792 28.5042) (end 83.156 27.976992) (width 0.2) (layer "F.Cu") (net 3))
 (segment (start 80.056 29.1292) (end 79.431 28.5042) (width 0.2) (layer "F.Cu") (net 3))
 (segment (start 83.156 26.531408) (end 80.703792 24.0792) (width 0.2) (layer "F.Cu") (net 3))
 (segment (start 80.703792 24.0792) (end 63.3416 24.0792) (width 0.2) (layer "F.Cu") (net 3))
 (segment (start 80.056 29.9542) (end 80.056 29.1292) (width 0.2) (layer "F.Cu") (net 3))
 (segment (start 53.1876 36.0172) (end 53.5178 36.0172) (width 0.2) (layer "F.Cu") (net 1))
 (segment (start 49.001248 37.7444) (end 45.5168 34.259952) (width 0.2) (layer "F.Cu") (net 1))
 (segment (start 43.2026 29.3596) (end 42.362 29.3596) (width 0.2) (layer "F.Cu") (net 1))
 (segment (start 42.362 26.8196) (end 42.016448 26.8196) (width 0.2) (layer "F.Cu") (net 1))
 (segment (start 47.0662 40.259) (end 49.5808 37.7444) (width 0.2) (layer "F.Cu") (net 1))
 (segment (start 45.5168 34.259952) (end 45.5168 31.6738) (width 0.2) (layer "F.Cu") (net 1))
 (segment (start 41.087 27.749048) (end 41.087 29.059599) (width 0.2) (layer "F.Cu") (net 1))
 (segment (start 53.5178 36.0172) (end 53.7718 35.7632) (width 0.2) (layer "F.Cu") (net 1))
 (segment (start 41.387001 29.3596) (end 42.362 29.3596) (width 0.2) (layer "F.Cu") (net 1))
 (segment (start 53.7718 35.7632) (end 55.6016 35.7632) (width 0.2) (layer "F.Cu") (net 1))
 (segment (start 49.5808 37.7444) (end 49.001248 37.7444) (width 0.2) (layer "F.Cu") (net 1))
 (segment (start 42.016448 26.8196) (end 41.087 27.749048) (width 0.2) (layer "F.Cu") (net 1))
 (segment (start 44.3738 40.259) (end 47.0662 40.259) (width 0.2) (layer "F.Cu") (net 1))
 (segment (start 45.5168 31.6738) (end 43.2026 29.3596) (width 0.2) (layer "F.Cu") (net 1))
 (segment (start 41.087 29.059599) (end 41.387001 29.3596) (width 0.2) (layer "F.Cu") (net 1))
 (via (at 53.1876 36.0172) (size 0.6) (drill 0.3) (layers "F.Cu" "B.Cu") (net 1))
 (via (at 49.5808 37.7444) (size 0.6) (drill 0.3) (layers "F.Cu" "B.Cu") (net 1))
 (segment (start 51.308 36.0172) (end 53.1876 36.0172) (width 0.2) (layer "B.Cu") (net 1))
 (segment (start 49.5808 37.7444) (end 51.308 36.0172) (width 0.2) (layer "B.Cu") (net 1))
 (segment (start 48.257552 31.2296) (end 45.847552 31.2296) (width 0.2) (layer "F.Cu") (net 6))
 (segment (start 57.0484 40.2082) (end 56.2734 40.9832) (width 0.2) (layer "F.Cu") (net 6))
 (segment (start 54.9786 40.9832) (end 48.587 34.5916) (width 0.2) (layer "F.Cu") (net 6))
 (segment (start 56.2734 40.9832) (end 54.9786 40.9832) (width 0.2) (layer "F.Cu") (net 6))
 (segment (start 42.707552 28.0896) (end 42.362 28.0896) (width 0.2) (layer "F.Cu") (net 6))
 (segment (start 48.587 34.5916) (end 48.587 31.559048) (width 0.2) (layer "F.Cu") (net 6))
 (segment (start 45.847552 31.2296) (end 42.707552 28.0896) (width 0.2) (layer "F.Cu") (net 6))
 (segment (start 48.587 31.559048) (end 48.257552 31.2296) (width 0.2) (layer "F.Cu") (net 6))
 (segment (start 41.0718 31.1912) (end 41.6334 30.6296) (width 0.2) (layer "F.Cu") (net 7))
 (segment (start 47.7396 45.7838) (end 41.0718 39.116) (width 0.2) (layer "F.Cu") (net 7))
 (segment (start 56.9214 45.0088) (end 56.1464 45.7838) (width 0.2) (layer "F.Cu") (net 7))
 (segment (start 41.6334 30.6296) (end 42.362 30.6296) (width 0.2) (layer "F.Cu") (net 7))
 (segment (start 56.1464 45.7838) (end 47.7396 45.7838) (width 0.2) (layer "F.Cu") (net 7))
 (segment (start 41.0718 39.116) (end 41.0718 31.1912) (width 0.2) (layer "F.Cu") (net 7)))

